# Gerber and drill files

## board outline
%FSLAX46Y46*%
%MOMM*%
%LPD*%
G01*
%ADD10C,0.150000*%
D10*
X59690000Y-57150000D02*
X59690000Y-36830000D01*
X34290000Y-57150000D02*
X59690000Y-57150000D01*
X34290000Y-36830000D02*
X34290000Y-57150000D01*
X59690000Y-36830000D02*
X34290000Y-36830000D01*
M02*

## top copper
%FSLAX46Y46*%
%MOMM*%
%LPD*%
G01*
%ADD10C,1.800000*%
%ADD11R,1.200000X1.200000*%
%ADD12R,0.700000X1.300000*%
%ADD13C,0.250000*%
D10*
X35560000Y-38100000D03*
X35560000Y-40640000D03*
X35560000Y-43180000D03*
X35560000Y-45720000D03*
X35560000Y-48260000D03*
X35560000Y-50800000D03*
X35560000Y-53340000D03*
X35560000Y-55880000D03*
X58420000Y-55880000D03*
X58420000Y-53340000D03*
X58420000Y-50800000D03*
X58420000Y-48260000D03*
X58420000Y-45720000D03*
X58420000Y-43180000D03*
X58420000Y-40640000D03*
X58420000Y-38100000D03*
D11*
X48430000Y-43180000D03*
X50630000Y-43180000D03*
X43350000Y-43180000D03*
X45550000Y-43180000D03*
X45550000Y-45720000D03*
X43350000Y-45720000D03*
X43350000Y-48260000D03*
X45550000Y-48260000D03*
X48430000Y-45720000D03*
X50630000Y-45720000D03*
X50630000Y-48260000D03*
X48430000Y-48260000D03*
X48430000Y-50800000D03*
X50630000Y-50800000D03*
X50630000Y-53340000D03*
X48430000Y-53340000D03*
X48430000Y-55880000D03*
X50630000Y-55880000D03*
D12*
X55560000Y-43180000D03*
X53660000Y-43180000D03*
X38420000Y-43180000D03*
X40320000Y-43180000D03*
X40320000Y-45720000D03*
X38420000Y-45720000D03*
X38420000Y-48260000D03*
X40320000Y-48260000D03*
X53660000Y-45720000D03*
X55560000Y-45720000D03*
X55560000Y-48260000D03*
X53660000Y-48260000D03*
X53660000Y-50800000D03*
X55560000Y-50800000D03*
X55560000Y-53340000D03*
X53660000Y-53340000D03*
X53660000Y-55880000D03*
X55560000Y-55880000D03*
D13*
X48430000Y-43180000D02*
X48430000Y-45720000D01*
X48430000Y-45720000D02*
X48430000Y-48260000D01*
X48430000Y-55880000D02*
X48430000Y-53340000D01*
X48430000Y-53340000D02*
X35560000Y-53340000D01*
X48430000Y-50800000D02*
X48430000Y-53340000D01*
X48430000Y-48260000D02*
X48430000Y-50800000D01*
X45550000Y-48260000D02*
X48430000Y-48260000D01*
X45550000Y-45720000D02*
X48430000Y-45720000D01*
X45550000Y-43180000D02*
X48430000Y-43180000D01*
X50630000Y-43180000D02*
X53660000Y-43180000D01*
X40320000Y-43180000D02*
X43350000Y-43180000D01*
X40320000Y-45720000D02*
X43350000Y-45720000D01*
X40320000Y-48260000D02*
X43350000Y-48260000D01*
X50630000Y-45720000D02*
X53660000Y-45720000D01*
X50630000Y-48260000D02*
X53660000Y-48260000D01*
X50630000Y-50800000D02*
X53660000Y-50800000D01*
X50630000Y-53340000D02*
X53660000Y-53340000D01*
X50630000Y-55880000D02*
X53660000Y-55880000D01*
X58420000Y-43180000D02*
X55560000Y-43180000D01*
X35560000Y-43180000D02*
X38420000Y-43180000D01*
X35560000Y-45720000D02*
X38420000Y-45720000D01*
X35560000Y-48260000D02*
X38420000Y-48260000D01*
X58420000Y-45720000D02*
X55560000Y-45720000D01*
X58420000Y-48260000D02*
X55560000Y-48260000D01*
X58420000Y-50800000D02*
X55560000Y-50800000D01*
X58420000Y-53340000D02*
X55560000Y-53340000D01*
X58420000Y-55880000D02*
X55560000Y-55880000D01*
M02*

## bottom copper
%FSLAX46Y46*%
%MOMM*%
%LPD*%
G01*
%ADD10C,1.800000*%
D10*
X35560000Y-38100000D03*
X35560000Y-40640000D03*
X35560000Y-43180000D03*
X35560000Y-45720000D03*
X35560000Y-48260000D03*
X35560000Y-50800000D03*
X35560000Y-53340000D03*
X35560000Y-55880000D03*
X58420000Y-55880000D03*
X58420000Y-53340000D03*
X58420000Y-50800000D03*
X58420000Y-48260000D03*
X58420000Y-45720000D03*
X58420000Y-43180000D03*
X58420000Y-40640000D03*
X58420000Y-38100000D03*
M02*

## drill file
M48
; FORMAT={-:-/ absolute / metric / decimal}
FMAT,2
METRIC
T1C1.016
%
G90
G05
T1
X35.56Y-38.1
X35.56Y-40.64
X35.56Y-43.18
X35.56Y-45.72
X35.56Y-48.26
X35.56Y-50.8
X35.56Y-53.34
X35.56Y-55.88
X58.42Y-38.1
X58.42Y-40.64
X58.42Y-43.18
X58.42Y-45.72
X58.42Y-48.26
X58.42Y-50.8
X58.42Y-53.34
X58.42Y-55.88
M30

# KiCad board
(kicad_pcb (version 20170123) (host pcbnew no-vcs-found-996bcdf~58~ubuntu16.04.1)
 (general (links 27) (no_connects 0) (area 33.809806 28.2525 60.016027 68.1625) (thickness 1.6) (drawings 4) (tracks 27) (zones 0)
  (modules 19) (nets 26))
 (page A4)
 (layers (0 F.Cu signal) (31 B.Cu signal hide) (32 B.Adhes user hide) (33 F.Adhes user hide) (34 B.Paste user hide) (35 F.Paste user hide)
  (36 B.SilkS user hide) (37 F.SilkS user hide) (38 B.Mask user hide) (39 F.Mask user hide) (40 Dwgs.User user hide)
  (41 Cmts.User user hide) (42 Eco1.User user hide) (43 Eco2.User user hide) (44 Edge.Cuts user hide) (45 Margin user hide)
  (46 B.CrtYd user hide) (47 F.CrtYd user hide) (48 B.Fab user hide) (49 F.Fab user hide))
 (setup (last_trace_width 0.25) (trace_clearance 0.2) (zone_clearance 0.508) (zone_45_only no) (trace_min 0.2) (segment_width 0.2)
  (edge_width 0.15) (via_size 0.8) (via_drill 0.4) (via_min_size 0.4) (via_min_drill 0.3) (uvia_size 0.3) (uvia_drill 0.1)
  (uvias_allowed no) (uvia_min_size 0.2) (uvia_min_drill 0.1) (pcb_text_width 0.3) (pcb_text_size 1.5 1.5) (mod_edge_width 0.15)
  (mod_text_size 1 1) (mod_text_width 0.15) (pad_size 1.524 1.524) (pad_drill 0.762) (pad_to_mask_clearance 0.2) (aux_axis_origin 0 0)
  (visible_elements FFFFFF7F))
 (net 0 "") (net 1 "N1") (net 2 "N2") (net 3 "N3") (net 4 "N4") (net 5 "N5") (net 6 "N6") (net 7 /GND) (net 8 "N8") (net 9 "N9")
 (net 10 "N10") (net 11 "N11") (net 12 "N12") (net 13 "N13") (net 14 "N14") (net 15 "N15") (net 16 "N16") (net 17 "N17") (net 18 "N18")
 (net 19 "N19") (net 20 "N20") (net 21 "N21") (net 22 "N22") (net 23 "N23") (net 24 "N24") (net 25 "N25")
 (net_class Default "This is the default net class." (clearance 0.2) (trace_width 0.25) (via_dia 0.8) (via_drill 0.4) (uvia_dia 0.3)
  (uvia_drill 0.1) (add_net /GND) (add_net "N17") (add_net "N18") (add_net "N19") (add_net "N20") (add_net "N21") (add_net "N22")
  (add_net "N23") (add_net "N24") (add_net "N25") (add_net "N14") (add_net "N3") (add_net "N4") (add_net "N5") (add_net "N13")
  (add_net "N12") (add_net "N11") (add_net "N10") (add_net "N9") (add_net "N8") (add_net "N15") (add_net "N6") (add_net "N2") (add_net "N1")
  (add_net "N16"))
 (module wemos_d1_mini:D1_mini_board (layer F.Cu) (at 46.99 48.26)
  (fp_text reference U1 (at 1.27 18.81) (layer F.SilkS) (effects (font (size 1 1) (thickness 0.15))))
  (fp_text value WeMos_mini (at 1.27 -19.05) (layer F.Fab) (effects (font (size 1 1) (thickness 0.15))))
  (pad 8 thru_hole circle (at -11.43 -10.16) (size 1.8 1.8) (drill 1.016) (layers *.Cu *.Mask F.SilkS) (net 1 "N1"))
  (pad 7 thru_hole circle (at -11.43 -7.62) (size 1.8 1.8) (drill 1.016) (layers *.Cu *.Mask F.SilkS) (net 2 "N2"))
  (pad 6 thru_hole circle (at -11.43 -5.08) (size 1.8 1.8) (drill 1.016) (layers *.Cu *.Mask F.SilkS) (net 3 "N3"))
  (pad 5 thru_hole circle (at -11.43 -2.54) (size 1.8 1.8) (drill 1.016) (layers *.Cu *.Mask F.SilkS) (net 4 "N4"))
  (pad 4 thru_hole circle (at -11.43 0) (size 1.8 1.8) (drill 1.016) (layers *.Cu *.Mask F.SilkS) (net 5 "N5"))
  (pad 3 thru_hole circle (at -11.43 2.54) (size 1.8 1.8) (drill 1.016) (layers *.Cu *.Mask F.SilkS) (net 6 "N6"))
  (pad 2 thru_hole circle (at -11.43 5.08) (size 1.8 1.8) (drill 1.016) (layers *.Cu *.Mask F.SilkS) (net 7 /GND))
  (pad 1 thru_hole circle (at -11.43 7.62) (size 1.8 1.8) (drill 1.016) (layers *.Cu *.Mask F.SilkS) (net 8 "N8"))
  (pad 16 thru_hole circle (at 11.43 7.62) (size 1.8 1.8) (drill 1.016) (layers *.Cu *.Mask F.SilkS) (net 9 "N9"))
  (pad 15 thru_hole circle (at 11.43 5.08) (size 1.8 1.8) (drill 1.016) (layers *.Cu *.Mask F.SilkS) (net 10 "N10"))
  (pad 14 thru_hole circle (at 11.43 2.54) (size 1.8 1.8) (drill 1.016) (layers *.Cu *.Mask F.SilkS) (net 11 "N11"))
  (pad 13 thru_hole circle (at 11.43 0) (size 1.8 1.8) (drill 1.016) (layers *.Cu *.Mask F.SilkS) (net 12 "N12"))
  (pad 12 thru_hole circle (at 11.43 -2.54) (size 1.8 1.8) (drill 1.016) (layers *.Cu *.Mask F.SilkS) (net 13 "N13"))
  (pad 11 thru_hole circle (at 11.43 -5.08) (size 1.8 1.8) (drill 1.016) (layers *.Cu *.Mask F.SilkS) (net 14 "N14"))
  (pad 10 thru_hole circle (at 11.43 -7.62) (size 1.8 1.8) (drill 1.016) (layers *.Cu *.Mask F.SilkS) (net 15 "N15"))
  (pad 9 thru_hole circle (at 11.43 -10.16) (size 1.8 1.8) (drill 1.016) (layers *.Cu *.Mask F.SilkS) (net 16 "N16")))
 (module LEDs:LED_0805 (layer F.Cu) (at 49.53 43.18)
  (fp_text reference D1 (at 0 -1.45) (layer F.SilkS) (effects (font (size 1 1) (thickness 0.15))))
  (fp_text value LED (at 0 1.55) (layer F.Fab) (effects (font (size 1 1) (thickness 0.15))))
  (pad 1 smd rect (at -1.1 0 180) (size 1.2 1.2) (layers F.Cu F.Paste F.Mask) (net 7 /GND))
  (pad 2 smd rect (at 1.1 0 180) (size 1.2 1.2) (layers F.Cu F.Paste F.Mask) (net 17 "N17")))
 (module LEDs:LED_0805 (layer F.Cu) (at 44.45 43.18 180)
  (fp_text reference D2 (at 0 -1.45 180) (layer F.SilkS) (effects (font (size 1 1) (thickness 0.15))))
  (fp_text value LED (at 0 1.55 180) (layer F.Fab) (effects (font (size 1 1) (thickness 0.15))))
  (pad 2 smd rect (at 1.1 0) (size 1.2 1.2) (layers F.Cu F.Paste F.Mask) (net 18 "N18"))
  (pad 1 smd rect (at -1.1 0) (size 1.2 1.2) (layers F.Cu F.Paste F.Mask) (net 7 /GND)))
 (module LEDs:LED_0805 (layer F.Cu) (at 44.45 45.72 180)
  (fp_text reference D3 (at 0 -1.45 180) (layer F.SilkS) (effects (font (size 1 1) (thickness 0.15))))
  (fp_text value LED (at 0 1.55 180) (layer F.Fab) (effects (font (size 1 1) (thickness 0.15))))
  (pad 1 smd rect (at -1.1 0) (size 1.2 1.2) (layers F.Cu F.Paste F.Mask) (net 7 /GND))
  (pad 2 smd rect (at 1.1 0) (size 1.2 1.2) (layers F.Cu F.Paste F.Mask) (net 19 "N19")))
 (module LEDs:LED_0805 (layer F.Cu) (at 44.45 48.26 180)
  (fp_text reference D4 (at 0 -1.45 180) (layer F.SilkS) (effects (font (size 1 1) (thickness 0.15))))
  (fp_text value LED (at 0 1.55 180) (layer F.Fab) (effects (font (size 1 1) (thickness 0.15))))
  (pad 2 smd rect (at 1.1 0) (size 1.2 1.2) (layers F.Cu F.Paste F.Mask) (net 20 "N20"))
  (pad 1 smd rect (at -1.1 0) (size 1.2 1.2) (layers F.Cu F.Paste F.Mask) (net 7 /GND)))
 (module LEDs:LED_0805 (layer F.Cu) (at 49.53 45.72)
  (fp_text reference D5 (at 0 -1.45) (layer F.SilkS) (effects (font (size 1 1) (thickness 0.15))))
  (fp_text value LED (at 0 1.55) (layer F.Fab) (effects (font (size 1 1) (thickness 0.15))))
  (pad 1 smd rect (at -1.1 0 180) (size 1.2 1.2) (layers F.Cu F.Paste F.Mask) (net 7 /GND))
  (pad 2 smd rect (at 1.1 0 180) (size 1.2 1.2) (layers F.Cu F.Paste F.Mask) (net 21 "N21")))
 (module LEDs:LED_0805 (layer F.Cu) (at 49.53 48.26)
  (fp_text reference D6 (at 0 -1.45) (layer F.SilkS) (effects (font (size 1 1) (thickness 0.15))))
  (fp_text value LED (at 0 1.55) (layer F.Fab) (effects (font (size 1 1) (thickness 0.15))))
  (pad 2 smd rect (at 1.1 0 180) (size 1.2 1.2) (layers F.Cu F.Paste F.Mask) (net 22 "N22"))
  (pad 1 smd rect (at -1.1 0 180) (size 1.2 1.2) (layers F.Cu F.Paste F.Mask) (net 7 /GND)))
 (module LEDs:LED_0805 (layer F.Cu) (at 49.53 50.8)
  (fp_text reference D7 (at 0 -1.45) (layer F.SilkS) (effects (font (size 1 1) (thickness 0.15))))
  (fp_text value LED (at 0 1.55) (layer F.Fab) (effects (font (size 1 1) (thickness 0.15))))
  (pad 1 smd rect (at -1.1 0 180) (size 1.2 1.2) (layers F.Cu F.Paste F.Mask) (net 7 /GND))
  (pad 2 smd rect (at 1.1 0 180) (size 1.2 1.2) (layers F.Cu F.Paste F.Mask) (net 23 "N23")))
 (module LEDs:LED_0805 (layer F.Cu) (at 49.53 53.34)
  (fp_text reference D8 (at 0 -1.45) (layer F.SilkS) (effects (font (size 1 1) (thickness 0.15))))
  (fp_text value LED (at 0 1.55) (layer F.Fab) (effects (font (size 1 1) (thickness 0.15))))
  (pad 2 smd rect (at 1.1 0 180) (size 1.2 1.2) (layers F.Cu F.Paste F.Mask) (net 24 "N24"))
  (pad 1 smd rect (at -1.1 0 180) (size 1.2 1.2) (layers F.Cu F.Paste F.Mask) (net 7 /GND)))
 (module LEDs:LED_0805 (layer F.Cu) (at 49.53 55.88)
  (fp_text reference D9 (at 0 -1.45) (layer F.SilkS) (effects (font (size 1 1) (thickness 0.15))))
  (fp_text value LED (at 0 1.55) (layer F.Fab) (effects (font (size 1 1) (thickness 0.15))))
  (pad 1 smd rect (at -1.1 0 180) (size 1.2 1.2) (layers F.Cu F.Paste F.Mask) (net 7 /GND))
  (pad 2 smd rect (at 1.1 0 180) (size 1.2 1.2) (layers F.Cu F.Paste F.Mask) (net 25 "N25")))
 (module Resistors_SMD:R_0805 (layer F.Cu) (at 54.61 43.18)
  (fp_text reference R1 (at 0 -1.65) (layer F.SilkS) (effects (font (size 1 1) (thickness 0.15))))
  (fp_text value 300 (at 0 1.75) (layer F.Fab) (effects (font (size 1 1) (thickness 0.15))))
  (pad 2 smd rect (at 0.95 0) (size 0.7 1.3) (layers F.Cu F.Paste F.Mask) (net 14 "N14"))
  (pad 1 smd rect (at -0.95 0) (size 0.7 1.3) (layers F.Cu F.Paste F.Mask) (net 17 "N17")))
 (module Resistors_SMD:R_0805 (layer F.Cu) (at 39.37 43.18)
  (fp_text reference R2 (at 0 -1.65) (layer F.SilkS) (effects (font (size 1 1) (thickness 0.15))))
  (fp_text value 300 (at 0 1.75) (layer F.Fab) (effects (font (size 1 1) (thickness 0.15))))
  (pad 1 smd rect (at -0.95 0) (size 0.7 1.3) (layers F.Cu F.Paste F.Mask) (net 3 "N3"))
  (pad 2 smd rect (at 0.95 0) (size 0.7 1.3) (layers F.Cu F.Paste F.Mask) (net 18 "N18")))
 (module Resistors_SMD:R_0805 (layer F.Cu) (at 39.37 45.72)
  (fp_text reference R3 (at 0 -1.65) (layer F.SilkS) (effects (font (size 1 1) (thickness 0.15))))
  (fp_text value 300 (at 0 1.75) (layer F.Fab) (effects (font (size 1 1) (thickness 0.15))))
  (pad 2 smd rect (at 0.95 0) (size 0.7 1.3) (layers F.Cu F.Paste F.Mask) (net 19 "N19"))
  (pad 1 smd rect (at -0.95 0) (size 0.7 1.3) (layers F.Cu F.Paste F.Mask) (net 4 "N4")))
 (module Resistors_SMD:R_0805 (layer F.Cu) (at 39.37 48.26)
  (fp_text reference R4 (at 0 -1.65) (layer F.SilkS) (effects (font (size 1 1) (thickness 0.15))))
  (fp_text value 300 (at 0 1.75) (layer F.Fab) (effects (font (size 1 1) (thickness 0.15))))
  (pad 1 smd rect (at -0.95 0) (size 0.7 1.3) (layers F.Cu F.Paste F.Mask) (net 5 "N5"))
  (pad 2 smd rect (at 0.95 0) (size 0.7 1.3) (layers F.Cu F.Paste F.Mask) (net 20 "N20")))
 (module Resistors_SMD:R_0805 (layer F.Cu) (at 54.61 45.72 180)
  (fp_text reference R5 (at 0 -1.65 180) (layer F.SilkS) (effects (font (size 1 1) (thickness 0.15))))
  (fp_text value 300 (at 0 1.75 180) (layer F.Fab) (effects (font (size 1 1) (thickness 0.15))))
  (pad 2 smd rect (at 0.95 0 180) (size 0.7 1.3) (layers F.Cu F.Paste F.Mask) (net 21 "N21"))
  (pad 1 smd rect (at -0.95 0 180) (size 0.7 1.3) (layers F.Cu F.Paste F.Mask) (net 13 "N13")))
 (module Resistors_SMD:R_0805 (layer F.Cu) (at 54.61 48.26 180)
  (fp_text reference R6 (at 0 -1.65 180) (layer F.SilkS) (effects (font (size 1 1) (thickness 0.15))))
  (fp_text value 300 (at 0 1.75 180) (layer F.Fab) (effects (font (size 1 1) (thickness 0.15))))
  (pad 1 smd rect (at -0.95 0 180) (size 0.7 1.3) (layers F.Cu F.Paste F.Mask) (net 12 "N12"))
  (pad 2 smd rect (at 0.95 0 180) (size 0.7 1.3) (layers F.Cu F.Paste F.Mask) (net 22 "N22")))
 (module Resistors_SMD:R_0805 (layer F.Cu) (at 54.61 50.8 180)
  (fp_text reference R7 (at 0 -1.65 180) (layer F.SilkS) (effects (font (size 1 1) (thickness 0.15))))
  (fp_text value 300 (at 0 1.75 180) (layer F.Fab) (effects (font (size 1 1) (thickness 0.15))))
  (pad 2 smd rect (at 0.95 0 180) (size 0.7 1.3) (layers F.Cu F.Paste F.Mask) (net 23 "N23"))
  (pad 1 smd rect (at -0.95 0 180) (size 0.7 1.3) (layers F.Cu F.Paste F.Mask) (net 11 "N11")))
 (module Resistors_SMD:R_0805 (layer F.Cu) (at 54.61 53.34 180)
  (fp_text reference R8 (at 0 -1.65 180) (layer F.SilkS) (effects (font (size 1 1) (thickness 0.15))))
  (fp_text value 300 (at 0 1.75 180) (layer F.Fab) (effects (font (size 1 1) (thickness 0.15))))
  (pad 1 smd rect (at -0.95 0 180) (size 0.7 1.3) (layers F.Cu F.Paste F.Mask) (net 10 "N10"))
  (pad 2 smd rect (at 0.95 0 180) (size 0.7 1.3) (layers F.Cu F.Paste F.Mask) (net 24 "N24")))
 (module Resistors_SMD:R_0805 (layer F.Cu) (at 54.61 55.88 180)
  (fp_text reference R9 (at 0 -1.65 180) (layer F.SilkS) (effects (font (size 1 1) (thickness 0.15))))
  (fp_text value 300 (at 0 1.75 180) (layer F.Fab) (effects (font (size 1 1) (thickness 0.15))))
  (pad 2 smd rect (at 0.95 0 180) (size 0.7 1.3) (layers F.Cu F.Paste F.Mask) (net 25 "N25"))
  (pad 1 smd rect (at -0.95 0 180) (size 0.7 1.3) (layers F.Cu F.Paste F.Mask) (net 9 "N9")))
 (gr_line (start 59.69 57.15) (end 59.69 36.83) (angle 90) (layer Edge.Cuts) (width 0.15))
 (gr_line (start 34.29 57.15) (end 59.69 57.15) (angle 90) (layer Edge.Cuts) (width 0.15))
 (gr_line (start 34.29 36.83) (end 34.29 57.15) (angle 90) (layer Edge.Cuts) (width 0.15))
 (gr_line (start 59.69 36.83) (end 34.29 36.83) (angle 90) (layer Edge.Cuts) (width 0.15))
 (segment (start 48.43 43.18) (end 48.43 45.72) (width 0.25) (layer F.Cu) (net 7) (status C00000))
 (segment (start 48.43 45.72) (end 48.43 48.26) (width 0.25) (layer F.Cu) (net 7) (status C00000))
 (segment (start 48.43 55.88) (end 48.43 53.34) (width 0.25) (layer F.Cu) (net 7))
 (segment (start 48.43 53.34) (end 35.56 53.34) (width 0.25) (layer F.Cu) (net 7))
 (segment (start 48.43 50.8) (end 48.43 53.34) (width 0.25) (layer F.Cu) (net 7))
 (segment (start 48.43 48.26) (end 48.43 50.8) (width 0.25) (layer F.Cu) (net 7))
 (segment (start 45.55 48.26) (end 48.43 48.26) (width 0.25) (layer F.Cu) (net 7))
 (segment (start 45.55 45.72) (end 48.43 45.72) (width 0.25) (layer F.Cu) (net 7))
 (segment (start 45.55 43.18) (end 48.43 43.18) (width 0.25) (layer F.Cu) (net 7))
 (segment (start 50.63 43.18) (end 53.66 43.18) (width 0.25) (layer F.Cu) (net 17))
 (segment (start 40.32 43.18) (end 43.35 43.18) (width 0.25) (layer F.Cu) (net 18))
 (segment (start 40.32 45.72) (end 43.35 45.72) (width 0.25) (layer F.Cu) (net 19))
 (segment (start 40.32 48.26) (end 43.35 48.26) (width 0.25) (layer F.Cu) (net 20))
 (segment (start 50.63 45.72) (end 53.66 45.72) (width 0.25) (layer F.Cu) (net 21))
 (segment (start 50.63 48.26) (end 53.66 48.26) (width 0.25) (layer F.Cu) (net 22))
 (segment (start 50.63 50.8) (end 53.66 50.8) (width 0.25) (layer F.Cu) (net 23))
 (segment (start 50.63 53.34) (end 53.66 53.34) (width 0.25) (layer F.Cu) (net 24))
 (segment (start 50.63 55.88) (end 53.66 55.88) (width 0.25) (layer F.Cu) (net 25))
 (segment (start 58.42 43.18) (end 55.56 43.18) (width 0.25) (layer F.Cu) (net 14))
 (segment (start 35.56 43.18) (end 38.42 43.18) (width 0.25) (layer F.Cu) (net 3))
 (segment (start 35.56 45.72) (end 38.42 45.72) (width 0.25) (layer F.Cu) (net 4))
 (segment (start 35.56 48.26) (end 38.42 48.26) (width 0.25) (layer F.Cu) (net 5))
 (segment (start 58.42 45.72) (end 55.56 45.72) (width 0.25) (layer F.Cu) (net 13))
 (segment (start 58.42 48.26) (end 55.56 48.26) (width 0.25) (layer F.Cu) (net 12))
 (segment (start 58.42 50.8) (end 55.56 50.8) (width 0.25) (layer F.Cu) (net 11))
 (segment (start 58.42 53.34) (end 55.56 53.34) (width 0.25) (layer F.Cu) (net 10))
 (segment (start 58.42 55.88) (end 55.56 55.88) (width 0.25) (layer F.Cu) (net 9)))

